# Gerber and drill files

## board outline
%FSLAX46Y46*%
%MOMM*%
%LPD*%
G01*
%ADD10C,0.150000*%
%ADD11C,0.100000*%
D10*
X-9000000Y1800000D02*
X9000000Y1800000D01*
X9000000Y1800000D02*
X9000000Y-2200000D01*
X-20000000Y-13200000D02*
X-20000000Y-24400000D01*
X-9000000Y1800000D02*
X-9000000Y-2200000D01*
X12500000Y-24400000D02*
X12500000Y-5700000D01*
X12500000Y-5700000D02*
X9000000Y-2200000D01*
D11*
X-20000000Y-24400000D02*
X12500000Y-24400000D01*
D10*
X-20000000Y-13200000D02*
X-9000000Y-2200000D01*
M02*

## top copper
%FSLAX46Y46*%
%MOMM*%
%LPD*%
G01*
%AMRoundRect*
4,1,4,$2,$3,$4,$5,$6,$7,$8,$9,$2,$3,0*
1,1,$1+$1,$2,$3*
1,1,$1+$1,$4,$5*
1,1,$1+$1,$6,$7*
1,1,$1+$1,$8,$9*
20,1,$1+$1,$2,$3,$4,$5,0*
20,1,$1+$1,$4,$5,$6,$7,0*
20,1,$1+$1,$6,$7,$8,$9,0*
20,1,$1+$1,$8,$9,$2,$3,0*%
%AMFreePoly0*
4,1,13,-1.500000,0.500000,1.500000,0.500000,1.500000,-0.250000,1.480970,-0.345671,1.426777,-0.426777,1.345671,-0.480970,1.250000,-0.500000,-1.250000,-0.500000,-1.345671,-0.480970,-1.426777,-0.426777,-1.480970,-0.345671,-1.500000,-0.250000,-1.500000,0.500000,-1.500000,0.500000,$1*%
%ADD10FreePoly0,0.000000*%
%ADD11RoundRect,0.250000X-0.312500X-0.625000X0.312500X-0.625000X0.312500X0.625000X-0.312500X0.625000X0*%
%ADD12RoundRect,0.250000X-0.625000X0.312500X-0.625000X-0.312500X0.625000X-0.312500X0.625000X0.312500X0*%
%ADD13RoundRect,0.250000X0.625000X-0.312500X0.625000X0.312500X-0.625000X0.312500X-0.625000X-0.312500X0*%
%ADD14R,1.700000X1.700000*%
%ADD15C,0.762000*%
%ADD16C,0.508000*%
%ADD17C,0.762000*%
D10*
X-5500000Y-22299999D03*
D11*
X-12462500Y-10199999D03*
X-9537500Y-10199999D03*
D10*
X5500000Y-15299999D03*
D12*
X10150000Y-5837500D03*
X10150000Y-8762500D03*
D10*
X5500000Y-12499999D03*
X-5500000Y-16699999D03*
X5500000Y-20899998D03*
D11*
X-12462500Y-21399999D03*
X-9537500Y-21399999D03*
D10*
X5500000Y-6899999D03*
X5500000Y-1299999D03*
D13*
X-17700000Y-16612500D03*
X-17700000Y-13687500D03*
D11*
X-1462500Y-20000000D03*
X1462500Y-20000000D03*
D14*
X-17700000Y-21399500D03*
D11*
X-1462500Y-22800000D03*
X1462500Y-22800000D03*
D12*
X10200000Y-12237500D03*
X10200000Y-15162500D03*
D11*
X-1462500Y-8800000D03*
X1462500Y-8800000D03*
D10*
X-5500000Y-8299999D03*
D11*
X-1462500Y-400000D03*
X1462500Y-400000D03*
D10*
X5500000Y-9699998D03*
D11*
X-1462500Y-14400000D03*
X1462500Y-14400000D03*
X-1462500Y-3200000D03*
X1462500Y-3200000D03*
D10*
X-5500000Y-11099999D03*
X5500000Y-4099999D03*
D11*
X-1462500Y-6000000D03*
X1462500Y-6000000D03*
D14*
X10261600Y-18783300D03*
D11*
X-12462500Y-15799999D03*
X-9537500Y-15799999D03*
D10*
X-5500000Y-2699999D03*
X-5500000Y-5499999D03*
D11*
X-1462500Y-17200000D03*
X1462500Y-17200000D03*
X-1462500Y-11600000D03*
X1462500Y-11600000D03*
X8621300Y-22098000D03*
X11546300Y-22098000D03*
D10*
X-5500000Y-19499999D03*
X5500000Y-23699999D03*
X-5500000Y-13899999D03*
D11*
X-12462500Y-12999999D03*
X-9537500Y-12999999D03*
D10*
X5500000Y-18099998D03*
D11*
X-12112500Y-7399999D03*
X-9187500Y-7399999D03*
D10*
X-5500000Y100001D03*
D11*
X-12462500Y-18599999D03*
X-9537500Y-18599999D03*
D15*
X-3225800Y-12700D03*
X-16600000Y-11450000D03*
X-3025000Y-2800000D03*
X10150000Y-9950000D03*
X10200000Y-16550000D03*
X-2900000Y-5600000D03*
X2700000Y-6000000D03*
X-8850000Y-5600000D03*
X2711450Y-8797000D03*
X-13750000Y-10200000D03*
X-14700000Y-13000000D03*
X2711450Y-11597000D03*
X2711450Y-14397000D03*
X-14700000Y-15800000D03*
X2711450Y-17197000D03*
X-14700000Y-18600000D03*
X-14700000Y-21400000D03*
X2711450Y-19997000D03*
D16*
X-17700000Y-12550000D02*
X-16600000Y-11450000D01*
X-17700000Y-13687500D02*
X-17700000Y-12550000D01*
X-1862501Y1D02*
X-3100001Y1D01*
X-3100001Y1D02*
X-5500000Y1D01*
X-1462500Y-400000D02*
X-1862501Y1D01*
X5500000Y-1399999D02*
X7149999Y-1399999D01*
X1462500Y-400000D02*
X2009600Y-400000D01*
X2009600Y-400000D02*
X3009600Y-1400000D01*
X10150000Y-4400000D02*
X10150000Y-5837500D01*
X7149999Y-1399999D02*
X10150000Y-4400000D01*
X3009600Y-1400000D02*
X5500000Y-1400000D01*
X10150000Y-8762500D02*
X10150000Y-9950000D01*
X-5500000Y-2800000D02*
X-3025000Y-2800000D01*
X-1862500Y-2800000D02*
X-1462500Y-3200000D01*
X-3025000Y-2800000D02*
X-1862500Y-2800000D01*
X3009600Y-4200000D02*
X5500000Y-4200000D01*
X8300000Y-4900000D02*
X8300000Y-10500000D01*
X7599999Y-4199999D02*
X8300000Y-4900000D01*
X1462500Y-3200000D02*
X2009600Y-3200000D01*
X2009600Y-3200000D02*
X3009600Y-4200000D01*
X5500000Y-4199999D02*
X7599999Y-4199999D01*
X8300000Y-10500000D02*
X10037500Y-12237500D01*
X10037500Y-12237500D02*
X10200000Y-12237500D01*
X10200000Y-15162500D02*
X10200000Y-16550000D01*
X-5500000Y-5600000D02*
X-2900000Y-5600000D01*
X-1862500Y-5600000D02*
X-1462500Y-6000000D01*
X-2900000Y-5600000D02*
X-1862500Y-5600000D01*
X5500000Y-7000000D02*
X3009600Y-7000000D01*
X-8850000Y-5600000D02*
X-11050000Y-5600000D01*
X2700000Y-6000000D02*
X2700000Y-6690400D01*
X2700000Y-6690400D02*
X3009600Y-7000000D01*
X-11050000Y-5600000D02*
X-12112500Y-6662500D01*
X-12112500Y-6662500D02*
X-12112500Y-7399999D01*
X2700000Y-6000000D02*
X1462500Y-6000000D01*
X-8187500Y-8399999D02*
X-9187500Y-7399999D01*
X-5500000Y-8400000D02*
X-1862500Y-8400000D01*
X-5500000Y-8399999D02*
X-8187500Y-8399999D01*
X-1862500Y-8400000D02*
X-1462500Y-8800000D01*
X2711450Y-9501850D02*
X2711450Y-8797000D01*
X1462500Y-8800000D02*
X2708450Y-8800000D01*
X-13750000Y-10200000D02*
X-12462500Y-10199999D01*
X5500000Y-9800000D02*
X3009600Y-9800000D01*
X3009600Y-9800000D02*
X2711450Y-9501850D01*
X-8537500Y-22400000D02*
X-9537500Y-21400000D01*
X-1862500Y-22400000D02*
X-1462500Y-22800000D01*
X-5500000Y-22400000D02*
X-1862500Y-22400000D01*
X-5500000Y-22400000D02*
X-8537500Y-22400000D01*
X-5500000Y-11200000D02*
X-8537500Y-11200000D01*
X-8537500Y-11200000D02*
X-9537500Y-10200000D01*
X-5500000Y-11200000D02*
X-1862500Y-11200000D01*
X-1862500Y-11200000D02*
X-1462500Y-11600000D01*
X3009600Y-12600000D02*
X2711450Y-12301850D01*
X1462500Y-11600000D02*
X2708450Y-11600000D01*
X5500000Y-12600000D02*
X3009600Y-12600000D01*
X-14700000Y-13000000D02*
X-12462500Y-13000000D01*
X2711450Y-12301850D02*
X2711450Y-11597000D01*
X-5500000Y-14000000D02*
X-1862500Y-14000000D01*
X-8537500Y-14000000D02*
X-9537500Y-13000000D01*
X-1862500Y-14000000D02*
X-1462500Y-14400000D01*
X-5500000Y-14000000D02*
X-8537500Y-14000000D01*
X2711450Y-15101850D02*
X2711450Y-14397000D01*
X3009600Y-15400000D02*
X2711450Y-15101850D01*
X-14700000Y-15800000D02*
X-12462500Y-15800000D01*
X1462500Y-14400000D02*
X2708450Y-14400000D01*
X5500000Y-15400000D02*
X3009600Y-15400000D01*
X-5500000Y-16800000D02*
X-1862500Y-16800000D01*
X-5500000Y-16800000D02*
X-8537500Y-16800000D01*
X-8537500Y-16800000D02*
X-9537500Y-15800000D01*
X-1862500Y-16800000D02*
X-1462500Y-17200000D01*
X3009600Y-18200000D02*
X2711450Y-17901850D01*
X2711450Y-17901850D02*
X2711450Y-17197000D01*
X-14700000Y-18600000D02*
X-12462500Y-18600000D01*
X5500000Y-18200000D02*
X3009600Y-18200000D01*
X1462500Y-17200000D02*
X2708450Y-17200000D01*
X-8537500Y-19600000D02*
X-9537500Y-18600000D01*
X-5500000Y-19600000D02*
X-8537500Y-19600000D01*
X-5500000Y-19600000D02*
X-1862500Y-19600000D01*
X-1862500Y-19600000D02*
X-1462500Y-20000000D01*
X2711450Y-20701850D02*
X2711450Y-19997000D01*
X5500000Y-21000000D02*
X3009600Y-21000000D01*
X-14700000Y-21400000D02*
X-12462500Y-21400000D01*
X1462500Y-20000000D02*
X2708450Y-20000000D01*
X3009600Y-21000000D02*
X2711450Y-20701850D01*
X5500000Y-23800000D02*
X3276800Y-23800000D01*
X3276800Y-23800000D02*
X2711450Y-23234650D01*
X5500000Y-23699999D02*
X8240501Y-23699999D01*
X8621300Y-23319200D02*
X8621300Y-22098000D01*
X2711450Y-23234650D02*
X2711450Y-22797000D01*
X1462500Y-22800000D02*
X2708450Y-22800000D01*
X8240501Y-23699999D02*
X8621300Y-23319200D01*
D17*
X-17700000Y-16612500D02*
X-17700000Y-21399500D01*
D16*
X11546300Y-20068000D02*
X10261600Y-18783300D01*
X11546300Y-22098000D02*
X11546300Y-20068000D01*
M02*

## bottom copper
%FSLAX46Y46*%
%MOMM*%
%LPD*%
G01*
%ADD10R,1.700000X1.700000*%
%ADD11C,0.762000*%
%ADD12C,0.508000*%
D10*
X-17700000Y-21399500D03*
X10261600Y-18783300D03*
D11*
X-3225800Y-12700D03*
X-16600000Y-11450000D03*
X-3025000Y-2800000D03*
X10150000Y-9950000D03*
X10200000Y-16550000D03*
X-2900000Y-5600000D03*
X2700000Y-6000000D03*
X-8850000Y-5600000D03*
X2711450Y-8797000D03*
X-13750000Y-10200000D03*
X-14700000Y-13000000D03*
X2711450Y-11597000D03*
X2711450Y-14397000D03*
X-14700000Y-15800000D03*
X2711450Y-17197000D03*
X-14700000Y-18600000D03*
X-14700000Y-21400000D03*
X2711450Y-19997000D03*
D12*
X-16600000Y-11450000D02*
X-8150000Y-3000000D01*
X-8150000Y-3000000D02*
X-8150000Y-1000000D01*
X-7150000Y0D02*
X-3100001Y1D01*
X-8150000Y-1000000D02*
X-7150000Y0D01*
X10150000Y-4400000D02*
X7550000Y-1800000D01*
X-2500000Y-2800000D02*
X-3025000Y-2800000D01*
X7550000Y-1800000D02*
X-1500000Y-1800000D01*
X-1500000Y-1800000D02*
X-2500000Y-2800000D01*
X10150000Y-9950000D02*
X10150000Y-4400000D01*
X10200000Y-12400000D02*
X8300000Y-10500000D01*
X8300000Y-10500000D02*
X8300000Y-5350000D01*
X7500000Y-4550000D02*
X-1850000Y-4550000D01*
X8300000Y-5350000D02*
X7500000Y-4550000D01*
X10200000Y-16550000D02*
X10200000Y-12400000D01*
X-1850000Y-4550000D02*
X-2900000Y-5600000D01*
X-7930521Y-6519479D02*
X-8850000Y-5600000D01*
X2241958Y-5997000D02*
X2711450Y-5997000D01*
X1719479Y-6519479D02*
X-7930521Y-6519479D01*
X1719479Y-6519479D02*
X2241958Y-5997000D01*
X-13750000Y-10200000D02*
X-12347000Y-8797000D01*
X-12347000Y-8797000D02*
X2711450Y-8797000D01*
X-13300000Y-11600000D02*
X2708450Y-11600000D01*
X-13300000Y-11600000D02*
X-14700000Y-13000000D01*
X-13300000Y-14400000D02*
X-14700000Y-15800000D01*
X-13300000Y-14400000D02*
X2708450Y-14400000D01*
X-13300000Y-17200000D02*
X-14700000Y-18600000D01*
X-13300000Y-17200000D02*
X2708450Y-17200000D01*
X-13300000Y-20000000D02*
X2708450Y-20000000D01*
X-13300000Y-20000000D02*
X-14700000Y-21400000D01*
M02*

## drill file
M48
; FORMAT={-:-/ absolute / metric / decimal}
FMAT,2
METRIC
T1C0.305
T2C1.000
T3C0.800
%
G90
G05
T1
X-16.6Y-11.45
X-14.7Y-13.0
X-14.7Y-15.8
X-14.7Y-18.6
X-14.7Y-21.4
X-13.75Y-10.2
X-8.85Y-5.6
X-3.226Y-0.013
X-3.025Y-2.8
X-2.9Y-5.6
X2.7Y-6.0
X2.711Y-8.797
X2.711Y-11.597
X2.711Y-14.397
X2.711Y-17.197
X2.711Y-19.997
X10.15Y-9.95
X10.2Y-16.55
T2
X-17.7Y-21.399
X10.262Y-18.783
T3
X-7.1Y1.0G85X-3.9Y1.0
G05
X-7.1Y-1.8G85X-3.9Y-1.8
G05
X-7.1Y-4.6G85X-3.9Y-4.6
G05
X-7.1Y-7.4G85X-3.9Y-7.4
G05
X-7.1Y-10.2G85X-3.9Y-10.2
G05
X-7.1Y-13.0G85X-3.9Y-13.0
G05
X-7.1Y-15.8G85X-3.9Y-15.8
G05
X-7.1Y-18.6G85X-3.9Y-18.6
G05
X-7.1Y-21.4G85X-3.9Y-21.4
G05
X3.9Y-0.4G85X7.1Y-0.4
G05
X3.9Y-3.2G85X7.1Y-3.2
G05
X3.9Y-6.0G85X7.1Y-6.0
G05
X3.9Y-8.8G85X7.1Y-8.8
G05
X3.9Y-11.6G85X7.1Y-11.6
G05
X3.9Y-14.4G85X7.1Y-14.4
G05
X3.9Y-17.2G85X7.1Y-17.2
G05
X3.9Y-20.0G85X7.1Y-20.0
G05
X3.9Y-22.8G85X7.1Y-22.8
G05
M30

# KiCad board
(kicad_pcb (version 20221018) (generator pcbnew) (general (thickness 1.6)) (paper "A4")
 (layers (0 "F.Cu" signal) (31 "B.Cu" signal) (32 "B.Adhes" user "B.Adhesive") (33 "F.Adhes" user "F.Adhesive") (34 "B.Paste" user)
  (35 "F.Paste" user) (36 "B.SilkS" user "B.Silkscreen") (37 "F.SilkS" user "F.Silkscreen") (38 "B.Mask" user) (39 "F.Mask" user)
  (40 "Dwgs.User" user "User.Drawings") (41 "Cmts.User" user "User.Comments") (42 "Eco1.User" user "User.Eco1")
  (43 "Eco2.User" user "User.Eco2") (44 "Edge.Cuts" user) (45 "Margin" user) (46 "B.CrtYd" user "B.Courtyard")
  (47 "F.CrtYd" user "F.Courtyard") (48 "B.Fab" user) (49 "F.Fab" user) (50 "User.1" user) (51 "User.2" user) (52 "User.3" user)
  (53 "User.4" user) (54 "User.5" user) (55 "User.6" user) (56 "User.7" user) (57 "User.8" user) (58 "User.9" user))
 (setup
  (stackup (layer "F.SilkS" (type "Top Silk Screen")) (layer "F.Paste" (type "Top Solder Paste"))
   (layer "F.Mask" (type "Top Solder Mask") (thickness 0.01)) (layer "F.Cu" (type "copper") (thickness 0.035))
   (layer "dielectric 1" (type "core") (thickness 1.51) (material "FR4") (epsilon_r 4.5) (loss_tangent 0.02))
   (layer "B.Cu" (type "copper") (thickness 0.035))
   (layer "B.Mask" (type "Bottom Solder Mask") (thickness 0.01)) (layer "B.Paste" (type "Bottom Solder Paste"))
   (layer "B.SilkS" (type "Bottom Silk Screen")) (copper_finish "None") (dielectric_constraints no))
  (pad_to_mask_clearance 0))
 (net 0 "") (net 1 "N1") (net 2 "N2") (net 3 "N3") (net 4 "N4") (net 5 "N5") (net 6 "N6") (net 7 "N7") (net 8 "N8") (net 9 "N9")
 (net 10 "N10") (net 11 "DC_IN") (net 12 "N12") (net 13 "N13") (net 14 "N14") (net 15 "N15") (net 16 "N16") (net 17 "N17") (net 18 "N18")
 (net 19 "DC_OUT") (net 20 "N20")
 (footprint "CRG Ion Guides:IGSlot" (layer "F.Cu") (at -5.5 21.399999)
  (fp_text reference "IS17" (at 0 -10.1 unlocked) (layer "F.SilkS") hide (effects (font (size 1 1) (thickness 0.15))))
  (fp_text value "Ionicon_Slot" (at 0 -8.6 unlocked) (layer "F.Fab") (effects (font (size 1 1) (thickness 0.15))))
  (pad "" np_thru_hole oval (at 0 0) (size 4 0.8) (drill oval 4 0.8) (layers "*.Mask"))
  (pad "1" smd roundrect (at 0 0.9) (size 3 1) (layers "F.Cu" "F.Mask") (roundrect_rratio 0.25) (chamfer_ratio 0)
   (chamfer top_left top_right) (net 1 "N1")))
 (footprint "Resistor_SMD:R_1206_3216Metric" (layer "F.Cu") (at -11 10.199999)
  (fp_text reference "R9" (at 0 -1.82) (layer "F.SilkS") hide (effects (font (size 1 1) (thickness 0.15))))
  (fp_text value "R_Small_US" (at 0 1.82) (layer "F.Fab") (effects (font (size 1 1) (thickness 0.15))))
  (pad "1" smd roundrect (at -1.4625 0) (size 1.125 1.75) (layers "F.Cu" "F.Paste" "F.Mask") (roundrect_rratio 0.2222222222) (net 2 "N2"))
  (pad "2" smd roundrect (at 1.4625 0) (size 1.125 1.75) (layers "F.Cu" "F.Paste" "F.Mask") (roundrect_rratio 0.2222222222) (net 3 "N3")))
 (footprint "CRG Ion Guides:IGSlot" (layer "F.Cu") (at 5.5 14.399999)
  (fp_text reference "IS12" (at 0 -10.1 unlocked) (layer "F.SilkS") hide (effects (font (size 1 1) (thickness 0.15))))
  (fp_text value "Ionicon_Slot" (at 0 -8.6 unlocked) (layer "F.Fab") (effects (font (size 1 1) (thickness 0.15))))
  (pad "" np_thru_hole oval (at 0 0) (size 4 0.8) (drill oval 4 0.8) (layers "*.Mask"))
  (pad "1" smd roundrect (at 0 0.9) (size 3 1) (layers "F.Cu" "F.Mask") (roundrect_rratio 0.25) (chamfer_ratio 0)
   (chamfer top_left top_right) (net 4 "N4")))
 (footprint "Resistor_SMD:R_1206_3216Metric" (layer "F.Cu") (at 10.15 7.3 -90)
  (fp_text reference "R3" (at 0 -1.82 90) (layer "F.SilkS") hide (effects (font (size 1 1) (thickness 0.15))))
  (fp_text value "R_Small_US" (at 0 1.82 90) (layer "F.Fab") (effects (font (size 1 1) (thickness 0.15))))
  (pad "1" smd roundrect (at -1.4625 0 270) (size 1.125 1.75) (layers "F.Cu" "F.Paste" "F.Mask") (roundrect_rratio 0.2222222222)
   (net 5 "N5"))
  (pad "2" smd roundrect (at 1.4625 0 270) (size 1.125 1.75) (layers "F.Cu" "F.Paste" "F.Mask") (roundrect_rratio 0.2222222222) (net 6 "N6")))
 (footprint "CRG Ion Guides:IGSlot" (layer "F.Cu") (at 5.5 11.599999)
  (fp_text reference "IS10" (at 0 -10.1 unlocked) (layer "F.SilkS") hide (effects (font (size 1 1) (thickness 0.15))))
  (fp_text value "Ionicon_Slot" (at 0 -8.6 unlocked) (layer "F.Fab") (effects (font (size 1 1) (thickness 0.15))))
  (pad "" np_thru_hole oval (at 0 0) (size 4 0.8) (drill oval 4 0.8) (layers "*.Mask"))
  (pad "1" smd roundrect (at 0 0.9) (size 3 1) (layers "F.Cu" "F.Mask") (roundrect_rratio 0.25) (chamfer_ratio 0)
   (chamfer top_left top_right) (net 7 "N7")))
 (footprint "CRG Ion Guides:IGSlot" (layer "F.Cu") (at -5.5 15.799999)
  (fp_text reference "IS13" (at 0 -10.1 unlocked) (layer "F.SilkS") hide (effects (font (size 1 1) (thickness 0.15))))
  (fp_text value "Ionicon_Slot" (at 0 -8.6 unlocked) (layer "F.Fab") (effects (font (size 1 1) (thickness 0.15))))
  (pad "" np_thru_hole oval (at 0 0) (size 4 0.8) (drill oval 4 0.8) (layers "*.Mask"))
  (pad "1" smd roundrect (at 0 0.9) (size 3 1) (layers "F.Cu" "F.Mask") (roundrect_rratio 0.25) (chamfer_ratio 0)
   (chamfer top_left top_right) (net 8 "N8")))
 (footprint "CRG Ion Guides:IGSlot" (layer "F.Cu") (at 5.5 19.999998)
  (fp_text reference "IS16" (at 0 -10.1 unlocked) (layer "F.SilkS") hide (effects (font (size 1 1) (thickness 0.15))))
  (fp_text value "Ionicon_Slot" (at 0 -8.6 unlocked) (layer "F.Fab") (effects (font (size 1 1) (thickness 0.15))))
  (pad "" np_thru_hole oval (at 0 0) (size 4 0.8) (drill oval 4 0.8) (layers "*.Mask"))
  (pad "1" smd roundrect (at 0 0.9) (size 3 1) (layers "F.Cu" "F.Mask") (roundrect_rratio 0.25) (chamfer_ratio 0)
   (chamfer top_left top_right) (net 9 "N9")))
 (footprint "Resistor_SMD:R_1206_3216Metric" (layer "F.Cu") (at -11 21.399999)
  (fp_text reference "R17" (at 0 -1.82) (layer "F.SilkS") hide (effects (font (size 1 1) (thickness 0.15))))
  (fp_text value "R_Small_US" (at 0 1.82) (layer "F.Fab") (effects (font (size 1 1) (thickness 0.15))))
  (pad "1" smd roundrect (at -1.4625 0) (size 1.125 1.75) (layers "F.Cu" "F.Paste" "F.Mask") (roundrect_rratio 0.2222222222) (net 9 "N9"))
  (pad "2" smd roundrect (at 1.4625 0) (size 1.125 1.75) (layers "F.Cu" "F.Paste" "F.Mask") (roundrect_rratio 0.2222222222) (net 1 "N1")))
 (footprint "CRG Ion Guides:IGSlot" (layer "F.Cu") (at 5.5 5.999999)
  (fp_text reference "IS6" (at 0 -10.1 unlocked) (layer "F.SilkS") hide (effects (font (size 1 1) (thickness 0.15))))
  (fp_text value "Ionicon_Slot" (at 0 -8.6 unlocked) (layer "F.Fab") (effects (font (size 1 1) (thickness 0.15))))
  (pad "" np_thru_hole oval (at 0 0) (size 4 0.8) (drill oval 4 0.8) (layers "*.Mask"))
  (pad "1" smd roundrect (at 0 0.9) (size 3 1) (layers "F.Cu" "F.Mask") (roundrect_rratio 0.25) (chamfer_ratio 0)
   (chamfer top_left top_right) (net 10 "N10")))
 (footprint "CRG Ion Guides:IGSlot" (layer "F.Cu") (at 5.5 0.399999)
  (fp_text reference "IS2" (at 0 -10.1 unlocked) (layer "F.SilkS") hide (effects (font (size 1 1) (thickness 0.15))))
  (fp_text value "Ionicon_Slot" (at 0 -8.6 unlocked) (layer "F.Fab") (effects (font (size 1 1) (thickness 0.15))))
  (pad "" np_thru_hole oval (at 0 0) (size 4 0.8) (drill oval 4 0.8) (layers "*.Mask"))
  (pad "1" smd roundrect (at 0 0.9) (size 3 1) (layers "F.Cu" "F.Mask") (roundrect_rratio 0.25) (chamfer_ratio 0)
   (chamfer top_left top_right) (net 5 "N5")))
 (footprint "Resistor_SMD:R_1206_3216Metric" (layer "F.Cu") (at -17.7 15.15 90)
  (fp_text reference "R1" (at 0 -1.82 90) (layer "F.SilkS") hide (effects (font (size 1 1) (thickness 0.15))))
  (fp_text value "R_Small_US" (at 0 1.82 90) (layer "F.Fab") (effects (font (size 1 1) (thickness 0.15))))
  (pad "1" smd roundrect (at -1.4625 0 90) (size 1.125 1.75) (layers "F.Cu" "F.Paste" "F.Mask") (roundrect_rratio 0.2222222222)
   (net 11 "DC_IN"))
  (pad "2" smd roundrect (at 1.4625 0 90) (size 1.125 1.75) (layers "F.Cu" "F.Paste" "F.Mask") (roundrect_rratio 0.2222222222)
   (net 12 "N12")))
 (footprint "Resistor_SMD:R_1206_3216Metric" (layer "F.Cu") (at 0 20)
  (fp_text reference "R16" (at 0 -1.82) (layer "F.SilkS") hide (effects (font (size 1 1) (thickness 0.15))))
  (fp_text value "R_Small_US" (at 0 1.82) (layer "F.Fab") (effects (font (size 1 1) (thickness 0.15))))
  (pad "1" smd roundrect (at -1.4625 0) (size 1.125 1.75) (layers "F.Cu" "F.Paste" "F.Mask") (roundrect_rratio 0.2222222222) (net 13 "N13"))
  (pad "2" smd roundrect (at 1.4625 0) (size 1.125 1.75) (layers "F.Cu" "F.Paste" "F.Mask") (roundrect_rratio 0.2222222222) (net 9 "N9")))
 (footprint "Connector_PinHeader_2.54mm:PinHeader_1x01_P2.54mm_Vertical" (layer "F.Cu") (at -17.7 21.3995 -90)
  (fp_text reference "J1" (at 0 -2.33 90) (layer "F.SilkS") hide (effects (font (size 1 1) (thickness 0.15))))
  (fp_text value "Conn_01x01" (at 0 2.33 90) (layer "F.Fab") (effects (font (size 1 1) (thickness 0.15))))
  (pad "1" thru_hole rect (at 0 0 270) (size 1.7 1.7) (drill 1) (layers "*.Cu" "*.Mask") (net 11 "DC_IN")))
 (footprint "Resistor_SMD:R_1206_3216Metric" (layer "F.Cu") (at 0 22.8)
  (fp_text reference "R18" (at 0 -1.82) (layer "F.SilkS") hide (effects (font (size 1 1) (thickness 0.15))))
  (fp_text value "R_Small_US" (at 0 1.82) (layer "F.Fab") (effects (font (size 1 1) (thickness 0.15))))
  (pad "1" smd roundrect (at -1.4625 0) (size 1.125 1.75) (layers "F.Cu" "F.Paste" "F.Mask") (roundrect_rratio 0.2222222222) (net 1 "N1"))
  (pad "2" smd roundrect (at 1.4625 0) (size 1.125 1.75) (layers "F.Cu" "F.Paste" "F.Mask") (roundrect_rratio 0.2222222222) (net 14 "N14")))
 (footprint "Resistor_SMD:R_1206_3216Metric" (layer "F.Cu") (at 10.2 13.7 -90)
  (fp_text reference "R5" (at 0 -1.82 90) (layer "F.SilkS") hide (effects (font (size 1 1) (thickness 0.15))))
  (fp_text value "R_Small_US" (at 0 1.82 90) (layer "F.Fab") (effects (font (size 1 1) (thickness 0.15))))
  (pad "1" smd roundrect (at -1.4625 0 270) (size 1.125 1.75) (layers "F.Cu" "F.Paste" "F.Mask") (roundrect_rratio 0.2222222222)
   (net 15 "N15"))
  (pad "2" smd roundrect (at 1.4625 0 270) (size 1.125 1.75) (layers "F.Cu" "F.Paste" "F.Mask") (roundrect_rratio 0.2222222222)
   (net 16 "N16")))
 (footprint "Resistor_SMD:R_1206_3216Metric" (layer "F.Cu") (at 0 8.8)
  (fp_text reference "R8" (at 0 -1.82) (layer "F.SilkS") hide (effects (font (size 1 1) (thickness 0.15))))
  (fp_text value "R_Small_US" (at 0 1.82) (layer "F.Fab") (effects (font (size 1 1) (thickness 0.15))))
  (pad "1" smd roundrect (at -1.4625 0) (size 1.125 1.75) (layers "F.Cu" "F.Paste" "F.Mask") (roundrect_rratio 0.2222222222) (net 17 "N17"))
  (pad "2" smd roundrect (at 1.4625 0) (size 1.125 1.75) (layers "F.Cu" "F.Paste" "F.Mask") (roundrect_rratio 0.2222222222) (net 2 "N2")))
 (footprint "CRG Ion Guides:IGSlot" (layer "F.Cu") (at -5.5 7.399999)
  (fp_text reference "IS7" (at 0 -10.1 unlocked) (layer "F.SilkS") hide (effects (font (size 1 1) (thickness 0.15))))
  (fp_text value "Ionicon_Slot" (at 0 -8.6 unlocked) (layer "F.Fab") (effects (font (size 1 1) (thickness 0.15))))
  (pad "" np_thru_hole oval (at 0 0) (size 4 0.8) (drill oval 4 0.8) (layers "*.Mask"))
  (pad "1" smd roundrect (at 0 0.9) (size 3 1) (layers "F.Cu" "F.Mask") (roundrect_rratio 0.25) (chamfer_ratio 0)
   (chamfer top_left top_right) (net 17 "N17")))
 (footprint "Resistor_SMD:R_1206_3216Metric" (layer "F.Cu") (at 0 0.4)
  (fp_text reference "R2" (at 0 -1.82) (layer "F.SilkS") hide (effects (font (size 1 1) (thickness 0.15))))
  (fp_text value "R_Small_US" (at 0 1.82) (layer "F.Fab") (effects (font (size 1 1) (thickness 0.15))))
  (pad "1" smd roundrect (at -1.4625 0) (size 1.125 1.75) (layers "F.Cu" "F.Paste" "F.Mask") (roundrect_rratio 0.2222222222) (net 12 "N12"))
  (pad "2" smd roundrect (at 1.4625 0) (size 1.125 1.75) (layers "F.Cu" "F.Paste" "F.Mask") (roundrect_rratio 0.2222222222) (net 5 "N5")))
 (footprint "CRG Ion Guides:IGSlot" (layer "F.Cu") (at 5.5 8.799998)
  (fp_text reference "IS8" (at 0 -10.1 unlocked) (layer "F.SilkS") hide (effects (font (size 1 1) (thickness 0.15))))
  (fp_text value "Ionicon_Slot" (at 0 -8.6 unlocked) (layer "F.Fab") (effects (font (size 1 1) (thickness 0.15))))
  (pad "" np_thru_hole oval (at 0 0) (size 4 0.8) (drill oval 4 0.8) (layers "*.Mask"))
  (pad "1" smd roundrect (at 0 0.9) (size 3 1) (layers "F.Cu" "F.Mask") (roundrect_rratio 0.25) (chamfer_ratio 0)
   (chamfer top_left top_right) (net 2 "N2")))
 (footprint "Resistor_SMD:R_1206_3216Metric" (layer "F.Cu") (at 0 14.4)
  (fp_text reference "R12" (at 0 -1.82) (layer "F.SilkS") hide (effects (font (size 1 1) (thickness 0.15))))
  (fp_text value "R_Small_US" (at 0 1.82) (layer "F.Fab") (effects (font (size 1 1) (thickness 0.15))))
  (pad "1" smd roundrect (at -1.4625 0) (size 1.125 1.75) (layers "F.Cu" "F.Paste" "F.Mask") (roundrect_rratio 0.2222222222) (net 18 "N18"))
  (pad "2" smd roundrect (at 1.4625 0) (size 1.125 1.75) (layers "F.Cu" "F.Paste" "F.Mask") (roundrect_rratio 0.2222222222) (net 4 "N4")))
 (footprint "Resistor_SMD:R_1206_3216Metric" (layer "F.Cu") (at 0 3.2)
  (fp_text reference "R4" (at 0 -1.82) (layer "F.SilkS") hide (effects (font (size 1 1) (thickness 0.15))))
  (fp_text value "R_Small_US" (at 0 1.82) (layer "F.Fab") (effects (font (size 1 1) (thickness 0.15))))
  (pad "1" smd roundrect (at -1.4625 0) (size 1.125 1.75) (layers "F.Cu" "F.Paste" "F.Mask") (roundrect_rratio 0.2222222222) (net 6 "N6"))
  (pad "2" smd roundrect (at 1.4625 0) (size 1.125 1.75) (layers "F.Cu" "F.Paste" "F.Mask") (roundrect_rratio 0.2222222222) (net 15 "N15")))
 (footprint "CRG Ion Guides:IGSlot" (layer "F.Cu") (at -5.5 10.199999)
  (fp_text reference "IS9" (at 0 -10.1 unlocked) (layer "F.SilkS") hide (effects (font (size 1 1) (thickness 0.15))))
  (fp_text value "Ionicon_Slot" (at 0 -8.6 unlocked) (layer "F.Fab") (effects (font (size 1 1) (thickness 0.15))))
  (pad "" np_thru_hole oval (at 0 0) (size 4 0.8) (drill oval 4 0.8) (layers "*.Mask"))
  (pad "1" smd roundrect (at 0 0.9) (size 3 1) (layers "F.Cu" "F.Mask") (roundrect_rratio 0.25) (chamfer_ratio 0)
   (chamfer top_left top_right) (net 3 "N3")))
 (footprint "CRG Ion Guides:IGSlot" (layer "F.Cu") (at 5.5 3.199999)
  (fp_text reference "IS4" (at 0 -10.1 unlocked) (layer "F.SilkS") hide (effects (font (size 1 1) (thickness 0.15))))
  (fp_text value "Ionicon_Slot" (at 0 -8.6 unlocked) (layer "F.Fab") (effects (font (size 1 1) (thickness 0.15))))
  (pad "" np_thru_hole oval (at 0 0) (size 4 0.8) (drill oval 4 0.8) (layers "*.Mask"))
  (pad "1" smd roundrect (at 0 0.9) (size 3 1) (layers "F.Cu" "F.Mask") (roundrect_rratio 0.25) (chamfer_ratio 0)
   (chamfer top_left top_right) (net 15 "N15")))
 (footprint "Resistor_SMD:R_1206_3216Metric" (layer "F.Cu") (at 0 6)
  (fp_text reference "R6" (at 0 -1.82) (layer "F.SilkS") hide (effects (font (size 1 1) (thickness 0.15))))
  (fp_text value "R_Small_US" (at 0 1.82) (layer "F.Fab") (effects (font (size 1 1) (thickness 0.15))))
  (pad "1" smd roundrect (at -1.4625 0) (size 1.125 1.75) (layers "F.Cu" "F.Paste" "F.Mask") (roundrect_rratio 0.2222222222) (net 16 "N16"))
  (pad "2" smd roundrect (at 1.4625 0) (size 1.125 1.75) (layers "F.Cu" "F.Paste" "F.Mask") (roundrect_rratio 0.2222222222) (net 10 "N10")))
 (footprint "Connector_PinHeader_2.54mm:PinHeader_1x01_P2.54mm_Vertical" (layer "F.Cu") (at 10.2616 18.7833 -90)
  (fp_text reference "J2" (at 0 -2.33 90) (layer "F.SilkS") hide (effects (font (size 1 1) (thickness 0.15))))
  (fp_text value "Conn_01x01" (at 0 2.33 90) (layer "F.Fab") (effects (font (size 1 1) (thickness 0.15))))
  (pad "1" thru_hole rect (at 0 0 270) (size 1.7 1.7) (drill 1) (layers "*.Cu" "*.Mask") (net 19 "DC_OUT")))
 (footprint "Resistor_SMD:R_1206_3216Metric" (layer "F.Cu") (at -11 15.799999)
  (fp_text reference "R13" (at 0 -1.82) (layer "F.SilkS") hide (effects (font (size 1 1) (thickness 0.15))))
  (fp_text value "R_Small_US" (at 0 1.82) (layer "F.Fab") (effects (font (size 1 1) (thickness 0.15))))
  (pad "1" smd roundrect (at -1.4625 0) (size 1.125 1.75) (layers "F.Cu" "F.Paste" "F.Mask") (roundrect_rratio 0.2222222222) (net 4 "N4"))
  (pad "2" smd roundrect (at 1.4625 0) (size 1.125 1.75) (layers "F.Cu" "F.Paste" "F.Mask") (roundrect_rratio 0.2222222222) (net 8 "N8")))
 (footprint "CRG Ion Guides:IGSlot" (layer "F.Cu") (at -5.5 1.799999)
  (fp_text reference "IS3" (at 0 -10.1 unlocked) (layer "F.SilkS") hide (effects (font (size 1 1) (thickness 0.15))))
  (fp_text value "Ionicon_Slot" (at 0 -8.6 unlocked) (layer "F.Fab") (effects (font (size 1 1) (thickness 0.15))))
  (pad "" np_thru_hole oval (at 0 0) (size 4 0.8) (drill oval 4 0.8) (layers "*.Mask"))
  (pad "1" smd roundrect (at 0 0.9) (size 3 1) (layers "F.Cu" "F.Mask") (roundrect_rratio 0.25) (chamfer_ratio 0)
   (chamfer top_left top_right) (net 6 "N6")))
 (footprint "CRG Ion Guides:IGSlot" (layer "F.Cu") (at -5.5 4.599999)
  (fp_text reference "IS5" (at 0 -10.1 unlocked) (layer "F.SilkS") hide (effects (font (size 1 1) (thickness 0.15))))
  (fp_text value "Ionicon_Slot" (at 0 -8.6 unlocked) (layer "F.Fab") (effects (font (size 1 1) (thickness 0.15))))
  (pad "" np_thru_hole oval (at 0 0) (size 4 0.8) (drill oval 4 0.8) (layers "*.Mask"))
  (pad "1" smd roundrect (at 0 0.9) (size 3 1) (layers "F.Cu" "F.Mask") (roundrect_rratio 0.25) (chamfer_ratio 0)
   (chamfer top_left top_right) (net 16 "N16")))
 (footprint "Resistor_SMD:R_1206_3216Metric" (layer "F.Cu") (at 0 17.2)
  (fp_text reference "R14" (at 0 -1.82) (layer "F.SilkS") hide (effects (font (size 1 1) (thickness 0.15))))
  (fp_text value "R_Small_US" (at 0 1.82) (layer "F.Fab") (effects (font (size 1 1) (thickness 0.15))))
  (pad "1" smd roundrect (at -1.4625 0) (size 1.125 1.75) (layers "F.Cu" "F.Paste" "F.Mask") (roundrect_rratio 0.2222222222) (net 8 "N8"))
  (pad "2" smd roundrect (at 1.4625 0) (size 1.125 1.75) (layers "F.Cu" "F.Paste" "F.Mask") (roundrect_rratio 0.2222222222) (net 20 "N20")))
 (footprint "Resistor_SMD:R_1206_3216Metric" (layer "F.Cu") (at 0 11.6)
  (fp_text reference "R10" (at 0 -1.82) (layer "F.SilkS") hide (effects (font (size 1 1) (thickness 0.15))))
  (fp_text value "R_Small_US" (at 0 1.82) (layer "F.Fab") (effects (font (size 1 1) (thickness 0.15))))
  (pad "1" smd roundrect (at -1.4625 0) (size 1.125 1.75) (layers "F.Cu" "F.Paste" "F.Mask") (roundrect_rratio 0.2222222222) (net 3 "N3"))
  (pad "2" smd roundrect (at 1.4625 0) (size 1.125 1.75) (layers "F.Cu" "F.Paste" "F.Mask") (roundrect_rratio 0.2222222222) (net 7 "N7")))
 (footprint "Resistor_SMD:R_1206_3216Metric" (layer "F.Cu") (at 10.0838 22.098)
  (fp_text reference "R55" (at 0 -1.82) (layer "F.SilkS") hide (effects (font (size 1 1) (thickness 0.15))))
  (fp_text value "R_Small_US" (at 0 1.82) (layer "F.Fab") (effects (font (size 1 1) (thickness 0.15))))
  (pad "1" smd roundrect (at -1.4625 0) (size 1.125 1.75) (layers "F.Cu" "F.Paste" "F.Mask") (roundrect_rratio 0.2222222222) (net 14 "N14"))
  (pad "2" smd roundrect (at 1.4625 0) (size 1.125 1.75) (layers "F.Cu" "F.Paste" "F.Mask") (roundrect_rratio 0.2222222222)
   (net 19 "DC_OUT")))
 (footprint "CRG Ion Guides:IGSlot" (layer "F.Cu") (at -5.5 18.599999)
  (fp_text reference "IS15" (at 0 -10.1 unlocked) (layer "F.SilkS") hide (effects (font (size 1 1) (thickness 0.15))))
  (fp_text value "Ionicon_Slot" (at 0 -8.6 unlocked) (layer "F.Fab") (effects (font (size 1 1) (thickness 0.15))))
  (pad "" np_thru_hole oval (at 0 0) (size 4 0.8) (drill oval 4 0.8) (layers "*.Mask"))
  (pad "1" smd roundrect (at 0 0.9) (size 3 1) (layers "F.Cu" "F.Mask") (roundrect_rratio 0.25) (chamfer_ratio 0)
   (chamfer top_left top_right) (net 13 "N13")))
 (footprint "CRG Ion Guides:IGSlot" (layer "F.Cu") (at 5.5 22.799999)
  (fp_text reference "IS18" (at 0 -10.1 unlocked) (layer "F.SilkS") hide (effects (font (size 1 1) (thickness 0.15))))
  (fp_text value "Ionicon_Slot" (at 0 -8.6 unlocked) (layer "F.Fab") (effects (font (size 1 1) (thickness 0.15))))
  (pad "" np_thru_hole oval (at 0 0) (size 4 0.8) (drill oval 4 0.8) (layers "*.Mask"))
  (pad "1" smd roundrect (at 0 0.9) (size 3 1) (layers "F.Cu" "F.Mask") (roundrect_rratio 0.25) (chamfer_ratio 0)
   (chamfer top_left top_right) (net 14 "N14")))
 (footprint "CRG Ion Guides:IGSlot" (layer "F.Cu") (at -5.5 12.999999)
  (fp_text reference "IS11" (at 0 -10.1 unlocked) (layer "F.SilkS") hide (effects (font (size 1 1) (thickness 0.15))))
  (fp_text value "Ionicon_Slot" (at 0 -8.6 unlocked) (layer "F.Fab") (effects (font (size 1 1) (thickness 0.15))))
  (pad "" np_thru_hole oval (at 0 0) (size 4 0.8) (drill oval 4 0.8) (layers "*.Mask"))
  (pad "1" smd roundrect (at 0 0.9) (size 3 1) (layers "F.Cu" "F.Mask") (roundrect_rratio 0.25) (chamfer_ratio 0)
   (chamfer top_left top_right) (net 18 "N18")))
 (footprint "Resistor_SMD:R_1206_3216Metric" (layer "F.Cu") (at -11 12.999999)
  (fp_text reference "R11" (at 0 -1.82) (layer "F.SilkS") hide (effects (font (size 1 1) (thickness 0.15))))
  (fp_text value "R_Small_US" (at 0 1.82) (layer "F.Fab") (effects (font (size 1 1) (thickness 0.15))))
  (pad "1" smd roundrect (at -1.4625 0) (size 1.125 1.75) (layers "F.Cu" "F.Paste" "F.Mask") (roundrect_rratio 0.2222222222) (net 7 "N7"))
  (pad "2" smd roundrect (at 1.4625 0) (size 1.125 1.75) (layers "F.Cu" "F.Paste" "F.Mask") (roundrect_rratio 0.2222222222) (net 18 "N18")))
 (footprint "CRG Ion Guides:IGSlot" (layer "F.Cu") (at 5.5 17.199998)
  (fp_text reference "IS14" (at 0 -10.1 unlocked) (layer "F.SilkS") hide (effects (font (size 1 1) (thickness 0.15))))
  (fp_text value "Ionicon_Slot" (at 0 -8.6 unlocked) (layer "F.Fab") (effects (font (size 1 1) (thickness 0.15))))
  (pad "" np_thru_hole oval (at 0 0) (size 4 0.8) (drill oval 4 0.8) (layers "*.Mask"))
  (pad "1" smd roundrect (at 0 0.9) (size 3 1) (layers "F.Cu" "F.Mask") (roundrect_rratio 0.25) (chamfer_ratio 0)
   (chamfer top_left top_right) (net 20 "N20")))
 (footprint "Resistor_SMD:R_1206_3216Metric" (layer "F.Cu") (at -10.65 7.399999)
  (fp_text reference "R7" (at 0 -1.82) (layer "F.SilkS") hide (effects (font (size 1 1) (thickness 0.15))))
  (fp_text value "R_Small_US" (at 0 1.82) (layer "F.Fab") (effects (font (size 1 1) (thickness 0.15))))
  (pad "1" smd roundrect (at -1.4625 0) (size 1.125 1.75) (layers "F.Cu" "F.Paste" "F.Mask") (roundrect_rratio 0.2222222222) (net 10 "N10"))
  (pad "2" smd roundrect (at 1.4625 0) (size 1.125 1.75) (layers "F.Cu" "F.Paste" "F.Mask") (roundrect_rratio 0.2222222222) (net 17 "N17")))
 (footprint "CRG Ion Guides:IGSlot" (layer "F.Cu") (at -5.5 -1.000001)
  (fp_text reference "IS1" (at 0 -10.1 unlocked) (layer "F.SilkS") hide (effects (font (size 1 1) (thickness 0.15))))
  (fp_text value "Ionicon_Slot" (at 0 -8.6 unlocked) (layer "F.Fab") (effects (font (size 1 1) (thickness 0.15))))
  (pad "" np_thru_hole oval (at 0 0) (size 4 0.8) (drill oval 4 0.8) (layers "*.Mask"))
  (pad "1" smd roundrect (at 0 0.9) (size 3 1) (layers "F.Cu" "F.Mask") (roundrect_rratio 0.25) (chamfer_ratio 0)
   (chamfer top_left top_right) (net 12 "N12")))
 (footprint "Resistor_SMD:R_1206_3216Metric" (layer "F.Cu") (at -11 18.599999)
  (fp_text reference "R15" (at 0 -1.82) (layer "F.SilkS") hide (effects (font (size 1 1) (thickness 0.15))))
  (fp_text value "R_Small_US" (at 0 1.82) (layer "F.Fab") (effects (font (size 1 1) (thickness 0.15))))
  (pad "1" smd roundrect (at -1.4625 0) (size 1.125 1.75) (layers "F.Cu" "F.Paste" "F.Mask") (roundrect_rratio 0.2222222222) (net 20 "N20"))
  (pad "2" smd roundrect (at 1.4625 0) (size 1.125 1.75) (layers "F.Cu" "F.Paste" "F.Mask") (roundrect_rratio 0.2222222222) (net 13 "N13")))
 (gr_line (start -9 -1.8) (end 9 -1.8) (stroke (width 0.15) (type solid)) (layer "Edge.Cuts"))
 (gr_line (start 9 -1.8) (end 9 2.2) (stroke (width 0.15) (type solid)) (layer "Edge.Cuts"))
 (gr_line (start -20 13.2) (end -20 24.4) (stroke (width 0.15) (type solid)) (layer "Edge.Cuts"))
 (gr_line (start -9 -1.8) (end -9 2.2) (stroke (width 0.15) (type solid)) (layer "Edge.Cuts"))
 (gr_line (start 12.5 24.4) (end 12.5 5.7) (stroke (width 0.15) (type solid)) (layer "Edge.Cuts"))
 (gr_line (start 12.5 5.7) (end 9 2.2) (stroke (width 0.15) (type solid)) (layer "Edge.Cuts"))
 (gr_line (start -20 24.4) (end 12.5 24.4) (stroke (width 0.1) (type solid)) (layer "Edge.Cuts"))
 (gr_line (start -20 13.2) (end -9 2.2) (stroke (width 0.15) (type solid)) (layer "Edge.Cuts"))
 (segment (start -17.7 12.55) (end -16.6 11.45) (width 0.508) (layer "F.Cu") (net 12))
 (segment (start -17.7 13.6875) (end -17.7 12.55) (width 0.508) (layer "F.Cu") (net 12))
 (segment (start -1.862501 -0.000001) (end -3.100001 -0.000001) (width 0.508) (layer "F.Cu") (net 12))
 (segment (start -3.100001 -0.000001) (end -5.5 -0.000001) (width 0.508) (layer "F.Cu") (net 12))
 (segment (start -1.4625 0.4) (end -1.862501 -0.000001) (width 0.508) (layer "F.Cu") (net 12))
 (via (at -3.2258 0.0127) (size 0.762) (drill 0.3048) (layers "F.Cu" "B.Cu") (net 12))
 (via (at -16.6 11.45) (size 0.762) (drill 0.3048) (layers "F.Cu" "B.Cu") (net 12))
 (segment (start -16.6 11.45) (end -8.15 3) (width 0.508) (layer "B.Cu") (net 12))
 (segment (start -8.15 3) (end -8.15 1) (width 0.508) (layer "B.Cu") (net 12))
 (segment (start -7.15 0) (end -3.100001 -0.000001) (width 0.508) (layer "B.Cu") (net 12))
 (segment (start -8.15 1) (end -7.15 0) (width 0.508) (layer "B.Cu") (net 12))
 (segment (start 5.5 1.399999) (end 7.149999 1.399999) (width 0.508) (layer "F.Cu") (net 5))
 (segment (start 1.4625 0.4) (end 2.0096 0.4) (width 0.508) (layer "F.Cu") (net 5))
 (segment (start 2.0096 0.4) (end 3.0096 1.4) (width 0.508) (layer "F.Cu") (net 5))
 (segment (start 10.15 4.4) (end 10.15 5.8375) (width 0.508) (layer "F.Cu") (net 5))
 (segment (start 7.149999 1.399999) (end 10.15 4.4) (width 0.508) (layer "F.Cu") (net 5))
 (segment (start 3.0096 1.4) (end 5.5 1.4) (width 0.508) (layer "F.Cu") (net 5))
 (segment (start 10.15 8.7625) (end 10.15 9.95) (width 0.508) (layer "F.Cu") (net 6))
 (segment (start -5.5 2.8) (end -3.025 2.8) (width 0.508) (layer "F.Cu") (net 6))
 (segment (start -1.8625 2.8) (end -1.4625 3.2) (width 0.508) (layer "F.Cu") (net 6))
 (segment (start -3.025 2.8) (end -1.8625 2.8) (width 0.508) (layer "F.Cu") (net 6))
 (via (at -3.025 2.8) (size 0.762) (drill 0.3048) (layers "F.Cu" "B.Cu") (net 6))
 (via (at 10.15 9.95) (size 0.762) (drill 0.3048) (layers "F.Cu" "B.Cu") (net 6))
 (segment (start 10.15 4.4) (end 7.55 1.8) (width 0.508) (layer "B.Cu") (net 6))
 (segment (start -2.5 2.8) (end -3.025 2.8) (width 0.508) (layer "B.Cu") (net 6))
 (segment (start 7.55 1.8) (end -1.5 1.8) (width 0.508) (layer "B.Cu") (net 6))
 (segment (start -1.5 1.8) (end -2.5 2.8) (width 0.508) (layer "B.Cu") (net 6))
 (segment (start 10.15 9.95) (end 10.15 4.4) (width 0.508) (layer "B.Cu") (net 6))
 (segment (start 3.0096 4.2) (end 5.5 4.2) (width 0.508) (layer "F.Cu") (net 15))
 (segment (start 8.3 4.9) (end 8.3 10.5) (width 0.508) (layer "F.Cu") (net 15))
 (segment (start 7.599999 4.199999) (end 8.3 4.9) (width 0.508) (layer "F.Cu") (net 15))
 (segment (start 1.4625 3.2) (end 2.0096 3.2) (width 0.508) (layer "F.Cu") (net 15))
 (segment (start 2.0096 3.2) (end 3.0096 4.2) (width 0.508) (layer "F.Cu") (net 15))
 (segment (start 5.5 4.199999) (end 7.599999 4.199999) (width 0.508) (layer "F.Cu") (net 15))
 (segment (start 8.3 10.5) (end 10.0375 12.2375) (width 0.508) (layer "F.Cu") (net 15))
 (segment (start 10.0375 12.2375) (end 10.2 12.2375) (width 0.508) (layer "F.Cu") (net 15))
 (segment (start 10.2 15.1625) (end 10.2 16.55) (width 0.508) (layer "F.Cu") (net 16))
 (segment (start -5.5 5.6) (end -2.9 5.6) (width 0.508) (layer "F.Cu") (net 16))
 (segment (start -1.8625 5.6) (end -1.4625 6) (width 0.508) (layer "F.Cu") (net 16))
 (segment (start -2.9 5.6) (end -1.8625 5.6) (width 0.508) (layer "F.Cu") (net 16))
 (via (at 10.2 16.55) (size 0.762) (drill 0.3048) (layers "F.Cu" "B.Cu") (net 16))
 (via (at -2.9 5.6) (size 0.762) (drill 0.3048) (layers "F.Cu" "B.Cu") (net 16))
 (segment (start 10.2 12.4) (end 8.3 10.5) (width 0.508) (layer "B.Cu") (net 16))
 (segment (start 8.3 10.5) (end 8.3 5.35) (width 0.508) (layer "B.Cu") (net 16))
 (segment (start 7.5 4.55) (end -1.85 4.55) (width 0.508) (layer "B.Cu") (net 16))
 (segment (start 8.3 5.35) (end 7.5 4.55) (width 0.508) (layer "B.Cu") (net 16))
 (segment (start 10.2 16.55) (end 10.2 12.4) (width 0.508) (layer "B.Cu") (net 16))
 (segment (start -1.85 4.55) (end -2.9 5.6) (width 0.508) (layer "B.Cu") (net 16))
 (segment (start 5.5 7) (end 3.0096 7) (width 0.508) (layer "F.Cu") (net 10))
 (segment (start -8.85 5.6) (end -11.05 5.6) (width 0.508) (layer "F.Cu") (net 10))
 (segment (start 2.7 6) (end 2.7 6.6904) (width 0.508) (layer "F.Cu") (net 10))
 (segment (start 2.7 6.6904) (end 3.0096 7) (width 0.508) (layer "F.Cu") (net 10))
 (segment (start -11.05 5.6) (end -12.1125 6.6625) (width 0.508) (layer "F.Cu") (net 10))
 (segment (start -12.1125 6.6625) (end -12.1125 7.399999) (width 0.508) (layer "F.Cu") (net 10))
 (segment (start 2.7 6) (end 1.4625 6) (width 0.508) (layer "F.Cu") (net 10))
 (via (at 2.7 6) (size 0.762) (drill 0.3048) (layers "F.Cu" "B.Cu") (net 10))
 (via (at -8.85 5.6) (size 0.762) (drill 0.3048) (layers "F.Cu" "B.Cu") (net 10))
 (segment (start -7.930521 6.519479) (end -8.85 5.6) (width 0.508) (layer "B.Cu") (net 10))
 (segment (start 2.241958 5.997) (end 2.71145 5.997) (width 0.508) (layer "B.Cu") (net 10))
 (segment (start 1.719479 6.519479) (end -7.930521 6.519479) (width 0.508) (layer "B.Cu") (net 10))
 (segment (start 1.719479 6.519479) (end 2.241958 5.997) (width 0.508) (layer "B.Cu") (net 10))
 (segment (start -8.1875 8.399999) (end -9.1875 7.399999) (width 0.508) (layer "F.Cu") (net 17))
 (segment (start -5.5 8.4) (end -1.8625 8.4) (width 0.508) (layer "F.Cu") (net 17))
 (segment (start -5.5 8.399999) (end -8.1875 8.399999) (width 0.508) (layer "F.Cu") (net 17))
 (segment (start -1.8625 8.4) (end -1.4625 8.8) (width 0.508) (layer "F.Cu") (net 17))
 (segment (start 2.71145 9.50185) (end 2.71145 8.797) (width 0.508) (layer "F.Cu") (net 2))
 (segment (start 1.4625 8.8) (end 2.70845 8.8) (width 0.508) (layer "F.Cu") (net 2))
 (segment (start -13.75 10.2) (end -12.4625 10.199999) (width 0.508) (layer "F.Cu") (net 2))
 (segment (start 5.5 9.8) (end 3.0096 9.8) (width 0.508) (layer "F.Cu") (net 2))
 (segment (start 3.0096 9.8) (end 2.71145 9.50185) (width 0.508) (layer "F.Cu") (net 2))
 (via (at 2.71145 8.797) (size 0.762) (drill 0.3048) (layers "F.Cu" "B.Cu") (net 2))
 (via (at -13.75 10.2) (size 0.762) (drill 0.3048) (layers "F.Cu" "B.Cu") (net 2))
 (segment (start -13.75 10.2) (end -12.347 8.797) (width 0.508) (layer "B.Cu") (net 2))
 (segment (start -12.347 8.797) (end 2.71145 8.797) (width 0.508) (layer "B.Cu") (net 2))
 (segment (start -8.5375 22.4) (end -9.5375 21.4) (width 0.508) (layer "F.Cu") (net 1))
 (segment (start -1.8625 22.4) (end -1.4625 22.8) (width 0.508) (layer "F.Cu") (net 1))
 (segment (start -5.5 22.4) (end -1.8625 22.4) (width 0.508) (layer "F.Cu") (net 1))
 (segment (start -5.5 22.4) (end -8.5375 22.4) (width 0.508) (layer "F.Cu") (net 1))
 (segment (start -5.5 11.2) (end -8.5375 11.2) (width 0.508) (layer "F.Cu") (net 3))
 (segment (start -8.5375 11.2) (end -9.5375 10.2) (width 0.508) (layer "F.Cu") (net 3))
 (segment (start -5.5 11.2) (end -1.8625 11.2) (width 0.508) (layer "F.Cu") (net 3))
 (segment (start -1.8625 11.2) (end -1.4625 11.6) (width 0.508) (layer "F.Cu") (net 3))
 (segment (start 3.0096 12.6) (end 2.71145 12.30185) (width 0.508) (layer "F.Cu") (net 7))
 (segment (start 1.4625 11.6) (end 2.70845 11.6) (width 0.508) (layer "F.Cu") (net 7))
 (segment (start 5.5 12.6) (end 3.0096 12.6) (width 0.508) (layer "F.Cu") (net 7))
 (segment (start -14.7 13) (end -12.4625 13) (width 0.508) (layer "F.Cu") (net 7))
 (segment (start 2.71145 12.30185) (end 2.71145 11.597) (width 0.508) (layer "F.Cu") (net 7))
 (via (at -14.7 13) (size 0.762) (drill 0.3048) (layers "F.Cu" "B.Cu") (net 7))
 (via (at 2.71145 11.597) (size 0.762) (drill 0.3048) (layers "F.Cu" "B.Cu") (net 7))
 (segment (start -13.3 11.6) (end 2.70845 11.6) (width 0.508) (layer "B.Cu") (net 7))
 (segment (start -13.3 11.6) (end -14.7 13) (width 0.508) (layer "B.Cu") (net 7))
 (segment (start -5.5 14) (end -1.8625 14) (width 0.508) (layer "F.Cu") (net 18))
 (segment (start -8.5375 14) (end -9.5375 13) (width 0.508) (layer "F.Cu") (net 18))
 (segment (start -1.8625 14) (end -1.4625 14.4) (width 0.508) (layer "F.Cu") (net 18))
 (segment (start -5.5 14) (end -8.5375 14) (width 0.508) (layer "F.Cu") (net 18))
 (segment (start 2.71145 15.10185) (end 2.71145 14.397) (width 0.508) (layer "F.Cu") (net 4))
 (segment (start 3.0096 15.4) (end 2.71145 15.10185) (width 0.508) (layer "F.Cu") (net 4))
 (segment (start -14.7 15.8) (end -12.4625 15.8) (width 0.508) (layer "F.Cu") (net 4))
 (segment (start 1.4625 14.4) (end 2.70845 14.4) (width 0.508) (layer "F.Cu") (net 4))
 (segment (start 5.5 15.4) (end 3.0096 15.4) (width 0.508) (layer "F.Cu") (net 4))
 (via (at 2.71145 14.397) (size 0.762) (drill 0.3048) (layers "F.Cu" "B.Cu") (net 4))
 (via (at -14.7 15.8) (size 0.762) (drill 0.3048) (layers "F.Cu" "B.Cu") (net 4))
 (segment (start -13.3 14.4) (end -14.7 15.8) (width 0.508) (layer "B.Cu") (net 4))
 (segment (start -13.3 14.4) (end 2.70845 14.4) (width 0.508) (layer "B.Cu") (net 4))
 (segment (start -5.5 16.8) (end -1.8625 16.8) (width 0.508) (layer "F.Cu") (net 8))
 (segment (start -5.5 16.8) (end -8.5375 16.8) (width 0.508) (layer "F.Cu") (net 8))
 (segment (start -8.5375 16.8) (end -9.5375 15.8) (width 0.508) (layer "F.Cu") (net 8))
 (segment (start -1.8625 16.8) (end -1.4625 17.2) (width 0.508) (layer "F.Cu") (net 8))
 (segment (start 3.0096 18.2) (end 2.71145 17.90185) (width 0.508) (layer "F.Cu") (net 20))
 (segment (start 2.71145 17.90185) (end 2.71145 17.197) (width 0.508) (layer "F.Cu") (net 20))
 (segment (start -14.7 18.6) (end -12.4625 18.6) (width 0.508) (layer "F.Cu") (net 20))
 (segment (start 5.5 18.2) (end 3.0096 18.2) (width 0.508) (layer "F.Cu") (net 20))
 (segment (start 1.4625 17.2) (end 2.70845 17.2) (width 0.508) (layer "F.Cu") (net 20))
 (via (at 2.71145 17.197) (size 0.762) (drill 0.3048) (layers "F.Cu" "B.Cu") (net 20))
 (via (at -14.7 18.6) (size 0.762) (drill 0.3048) (layers "F.Cu" "B.Cu") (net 20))
 (segment (start -13.3 17.2) (end -14.7 18.6) (width 0.508) (layer "B.Cu") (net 20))
 (segment (start -13.3 17.2) (end 2.70845 17.2) (width 0.508) (layer "B.Cu") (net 20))
 (segment (start -8.5375 19.6) (end -9.5375 18.6) (width 0.508) (layer "F.Cu") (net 13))
 (segment (start -5.5 19.6) (end -8.5375 19.6) (width 0.508) (layer "F.Cu") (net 13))
 (segment (start -5.5 19.6) (end -1.8625 19.6) (width 0.508) (layer "F.Cu") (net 13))
 (segment (start -1.8625 19.6) (end -1.4625 20) (width 0.508) (layer "F.Cu") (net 13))
 (segment (start 2.71145 20.70185) (end 2.71145 19.997) (width 0.508) (layer "F.Cu") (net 9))
 (segment (start 5.5 21) (end 3.0096 21) (width 0.508) (layer "F.Cu") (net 9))
 (segment (start -14.7 21.4) (end -12.4625 21.4) (width 0.508) (layer "F.Cu") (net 9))
 (segment (start 1.4625 20) (end 2.70845 20) (width 0.508) (layer "F.Cu") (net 9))
 (segment (start 3.0096 21) (end 2.71145 20.70185) (width 0.508) (layer "F.Cu") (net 9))
 (via (at -14.7 21.4) (size 0.762) (drill 0.3048) (layers "F.Cu" "B.Cu") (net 9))
 (via (at 2.71145 19.997) (size 0.762) (drill 0.3048) (layers "F.Cu" "B.Cu") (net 9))
 (segment (start -13.3 20) (end 2.70845 20) (width 0.508) (layer "B.Cu") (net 9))
 (segment (start -13.3 20) (end -14.7 21.4) (width 0.508) (layer "B.Cu") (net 9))
 (segment (start 5.5 23.8) (end 3.2768 23.8) (width 0.508) (layer "F.Cu") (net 14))
 (segment (start 3.2768 23.8) (end 2.71145 23.23465) (width 0.508) (layer "F.Cu") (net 14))
 (segment (start 5.5 23.699999) (end 8.240501 23.699999) (width 0.508) (layer "F.Cu") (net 14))
 (segment (start 8.6213 23.3192) (end 8.6213 22.098) (width 0.508) (layer "F.Cu") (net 14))
 (segment (start 2.71145 23.23465) (end 2.71145 22.797) (width 0.508) (layer "F.Cu") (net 14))
 (segment (start 1.4625 22.8) (end 2.70845 22.8) (width 0.508) (layer "F.Cu") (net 14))
 (segment (start 8.240501 23.699999) (end 8.6213 23.3192) (width 0.508) (layer "F.Cu") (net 14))
 (segment (start -17.7 16.6125) (end -17.7 21.3995) (width 0.762) (layer "F.Cu") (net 11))
 (segment (start 11.5463 20.068) (end 10.2616 18.7833) (width 0.508) (layer "F.Cu") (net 19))
 (segment (start 11.5463 22.098) (end 11.5463 20.068) (width 0.508) (layer "F.Cu") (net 19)))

